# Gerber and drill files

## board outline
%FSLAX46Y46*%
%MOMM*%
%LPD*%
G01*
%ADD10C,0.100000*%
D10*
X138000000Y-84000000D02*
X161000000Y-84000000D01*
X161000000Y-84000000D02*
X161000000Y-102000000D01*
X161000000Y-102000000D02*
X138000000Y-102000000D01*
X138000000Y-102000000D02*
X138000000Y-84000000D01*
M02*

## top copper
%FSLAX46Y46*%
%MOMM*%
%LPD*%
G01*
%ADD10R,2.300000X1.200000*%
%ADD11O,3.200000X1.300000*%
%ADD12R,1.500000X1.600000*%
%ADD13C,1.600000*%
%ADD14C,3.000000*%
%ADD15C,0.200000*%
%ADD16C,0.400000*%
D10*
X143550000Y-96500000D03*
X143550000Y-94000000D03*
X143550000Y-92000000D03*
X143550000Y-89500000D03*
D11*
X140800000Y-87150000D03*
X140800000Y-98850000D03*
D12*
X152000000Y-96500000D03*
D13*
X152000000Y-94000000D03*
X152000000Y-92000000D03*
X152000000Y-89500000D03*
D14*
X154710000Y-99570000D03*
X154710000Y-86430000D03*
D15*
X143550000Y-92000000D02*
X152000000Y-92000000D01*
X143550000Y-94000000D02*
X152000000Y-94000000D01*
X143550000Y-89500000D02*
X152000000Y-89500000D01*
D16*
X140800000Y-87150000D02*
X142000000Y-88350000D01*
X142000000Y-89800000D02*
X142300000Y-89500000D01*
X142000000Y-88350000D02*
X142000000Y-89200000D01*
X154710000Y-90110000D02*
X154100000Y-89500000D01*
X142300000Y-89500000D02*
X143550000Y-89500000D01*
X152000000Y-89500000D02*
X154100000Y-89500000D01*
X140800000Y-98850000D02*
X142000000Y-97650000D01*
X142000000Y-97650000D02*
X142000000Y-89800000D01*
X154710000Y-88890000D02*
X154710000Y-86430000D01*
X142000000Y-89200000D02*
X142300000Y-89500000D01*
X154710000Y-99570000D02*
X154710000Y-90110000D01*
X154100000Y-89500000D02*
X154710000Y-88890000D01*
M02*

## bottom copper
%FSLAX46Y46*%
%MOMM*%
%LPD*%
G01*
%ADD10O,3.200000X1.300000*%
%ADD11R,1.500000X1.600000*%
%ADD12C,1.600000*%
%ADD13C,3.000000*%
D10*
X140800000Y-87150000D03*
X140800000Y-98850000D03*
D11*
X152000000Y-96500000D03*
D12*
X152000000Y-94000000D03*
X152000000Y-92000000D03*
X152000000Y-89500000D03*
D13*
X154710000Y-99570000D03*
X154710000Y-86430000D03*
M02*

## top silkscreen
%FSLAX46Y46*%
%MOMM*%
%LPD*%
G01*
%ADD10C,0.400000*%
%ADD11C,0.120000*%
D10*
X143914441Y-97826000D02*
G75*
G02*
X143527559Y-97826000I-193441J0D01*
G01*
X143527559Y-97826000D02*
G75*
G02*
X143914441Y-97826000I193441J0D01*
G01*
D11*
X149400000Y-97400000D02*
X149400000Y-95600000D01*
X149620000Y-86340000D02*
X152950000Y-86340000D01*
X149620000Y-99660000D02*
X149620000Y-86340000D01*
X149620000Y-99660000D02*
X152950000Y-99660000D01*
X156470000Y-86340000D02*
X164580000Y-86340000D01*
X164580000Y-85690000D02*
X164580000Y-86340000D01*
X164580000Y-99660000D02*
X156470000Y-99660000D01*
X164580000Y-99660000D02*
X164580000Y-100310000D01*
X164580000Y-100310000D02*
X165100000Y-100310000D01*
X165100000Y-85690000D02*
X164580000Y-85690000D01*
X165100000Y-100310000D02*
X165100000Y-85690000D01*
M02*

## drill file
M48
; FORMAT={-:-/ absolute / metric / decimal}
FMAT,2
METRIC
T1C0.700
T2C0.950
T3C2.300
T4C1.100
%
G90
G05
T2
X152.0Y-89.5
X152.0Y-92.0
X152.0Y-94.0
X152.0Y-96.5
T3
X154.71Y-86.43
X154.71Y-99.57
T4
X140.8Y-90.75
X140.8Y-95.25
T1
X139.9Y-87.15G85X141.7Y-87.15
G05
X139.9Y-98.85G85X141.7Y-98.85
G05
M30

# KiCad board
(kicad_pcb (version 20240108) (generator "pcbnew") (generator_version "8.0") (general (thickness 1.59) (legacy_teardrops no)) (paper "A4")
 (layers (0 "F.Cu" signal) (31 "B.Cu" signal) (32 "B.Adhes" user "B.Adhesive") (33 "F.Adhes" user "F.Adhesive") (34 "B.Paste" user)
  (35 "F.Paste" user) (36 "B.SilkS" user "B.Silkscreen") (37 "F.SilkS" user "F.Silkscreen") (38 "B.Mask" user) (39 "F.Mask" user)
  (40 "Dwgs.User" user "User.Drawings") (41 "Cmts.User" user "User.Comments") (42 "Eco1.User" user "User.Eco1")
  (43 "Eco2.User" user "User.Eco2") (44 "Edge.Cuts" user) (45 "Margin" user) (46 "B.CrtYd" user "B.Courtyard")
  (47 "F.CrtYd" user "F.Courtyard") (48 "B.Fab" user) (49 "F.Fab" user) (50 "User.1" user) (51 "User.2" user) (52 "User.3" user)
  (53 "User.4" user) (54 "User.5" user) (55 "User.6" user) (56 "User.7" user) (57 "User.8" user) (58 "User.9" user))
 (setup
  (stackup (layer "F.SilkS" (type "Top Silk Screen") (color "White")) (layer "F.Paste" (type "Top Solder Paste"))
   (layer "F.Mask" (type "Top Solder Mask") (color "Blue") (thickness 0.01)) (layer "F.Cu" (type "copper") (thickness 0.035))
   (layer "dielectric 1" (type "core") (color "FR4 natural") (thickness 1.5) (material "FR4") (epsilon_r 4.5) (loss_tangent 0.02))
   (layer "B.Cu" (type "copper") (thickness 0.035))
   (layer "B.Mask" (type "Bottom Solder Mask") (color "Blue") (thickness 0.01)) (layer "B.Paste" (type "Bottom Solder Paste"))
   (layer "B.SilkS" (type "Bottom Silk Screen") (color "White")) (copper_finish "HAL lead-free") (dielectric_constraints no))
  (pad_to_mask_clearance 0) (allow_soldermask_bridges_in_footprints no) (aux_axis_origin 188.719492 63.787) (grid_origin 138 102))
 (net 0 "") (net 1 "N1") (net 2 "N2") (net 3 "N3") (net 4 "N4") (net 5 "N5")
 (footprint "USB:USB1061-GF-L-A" (layer "F.Cu") (at 140.8 93 -90)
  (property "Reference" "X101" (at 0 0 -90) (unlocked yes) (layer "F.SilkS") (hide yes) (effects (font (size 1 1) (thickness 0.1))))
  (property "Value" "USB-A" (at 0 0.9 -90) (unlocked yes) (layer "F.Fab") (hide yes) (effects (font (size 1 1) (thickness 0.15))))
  (fp_circle (center 4.826 -2.921) (end 5.019441 -2.921) (stroke (width 0.4) (type solid)) (fill none) (layer "F.SilkS"))
  (pad "" np_thru_hole circle (at -2.25 0 270) (size 1.1 1.1) (drill 1.1) (layers "*.Cu" "*.Mask"))
  (pad "" np_thru_hole circle (at 2.25 0 270) (size 1.1 1.1) (drill 1.1) (layers "*.Cu" "*.Mask"))
  (pad "1" smd rect (at 3.5 -2.75 270) (size 1.2 2.3) (layers "F.Cu" "F.Paste" "F.Mask") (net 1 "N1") (solder_mask_margin 0.102))
  (pad "2" smd rect (at 1 -2.75 270) (size 1.2 2.3) (layers "F.Cu" "F.Paste" "F.Mask") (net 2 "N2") (solder_mask_margin 0.102))
  (pad "3" smd rect (at -1 -2.75 270) (size 1.2 2.3) (layers "F.Cu" "F.Paste" "F.Mask") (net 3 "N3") (solder_mask_margin 0.102))
  (pad "4" smd rect (at -3.5 -2.75 270) (size 1.2 2.3) (layers "F.Cu" "F.Paste" "F.Mask") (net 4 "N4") (solder_mask_margin 0.102))
  (pad "5" thru_hole oval (at -5.85 0) (size 3.2 1.3) (drill oval 2.5 0.7) (layers "*.Cu" "*.Mask") (remove_unused_layers no) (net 4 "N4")
   (thermal_bridge_angle 45))
  (pad "5" thru_hole oval (at 5.85 0) (size 3.2 1.3) (drill oval 2.5 0.7) (layers "*.Cu" "*.Mask") (remove_unused_layers no) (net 4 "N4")
   (thermal_bridge_angle 45)))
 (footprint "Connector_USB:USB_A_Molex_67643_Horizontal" (layer "F.Cu") (at 152 96.5 90)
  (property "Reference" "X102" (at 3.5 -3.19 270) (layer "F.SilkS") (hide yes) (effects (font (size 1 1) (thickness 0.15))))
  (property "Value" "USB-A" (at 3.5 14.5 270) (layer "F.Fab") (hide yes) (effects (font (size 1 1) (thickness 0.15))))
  (fp_line (start -0.9 -2.6) (end 0.9 -2.6) (stroke (width 0.12) (type solid)) (layer "F.SilkS"))
  (fp_line (start 10.16 -2.38) (end 10.16 0.95) (stroke (width 0.12) (type solid)) (layer "F.SilkS"))
  (fp_line (start -3.16 -2.38) (end 10.16 -2.38) (stroke (width 0.12) (type solid)) (layer "F.SilkS"))
  (fp_line (start -3.16 -2.38) (end -3.16 0.95) (stroke (width 0.12) (type solid)) (layer "F.SilkS"))
  (fp_line (start 10.16 4.47) (end 10.16 12.58) (stroke (width 0.12) (type solid)) (layer "F.SilkS"))
  (fp_line (start 10.81 12.58) (end 10.16 12.58) (stroke (width 0.12) (type solid)) (layer "F.SilkS"))
  (fp_line (start -3.16 12.58) (end -3.16 4.47) (stroke (width 0.12) (type solid)) (layer "F.SilkS"))
  (fp_line (start -3.16 12.58) (end -3.81 12.58) (stroke (width 0.12) (type solid)) (layer "F.SilkS"))
  (fp_line (start -3.81 12.58) (end -3.81 13.1) (stroke (width 0.12) (type solid)) (layer "F.SilkS"))
  (fp_line (start 10.81 13.1) (end 10.81 12.58) (stroke (width 0.12) (type solid)) (layer "F.SilkS"))
  (fp_line (start -3.81 13.1) (end 10.81 13.1) (stroke (width 0.12) (type solid)) (layer "F.SilkS"))
  (pad "1" thru_hole rect (at 0 0 90) (size 1.6 1.5) (drill 0.95) (layers "*.Cu" "*.Mask") (remove_unused_layers no) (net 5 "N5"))
  (pad "2" thru_hole circle (at 2.5 0 90) (size 1.6 1.6) (drill 0.95) (layers "*.Cu" "*.Mask") (remove_unused_layers no) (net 2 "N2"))
  (pad "3" thru_hole circle (at 4.5 0 90) (size 1.6 1.6) (drill 0.95) (layers "*.Cu" "*.Mask") (remove_unused_layers no) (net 3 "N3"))
  (pad "4" thru_hole circle (at 7 0 90) (size 1.6 1.6) (drill 0.95) (layers "*.Cu" "*.Mask") (remove_unused_layers no) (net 4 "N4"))
  (pad "5" thru_hole circle (at -3.07 2.71 90) (size 3 3) (drill 2.3) (layers "*.Cu" "*.Mask") (remove_unused_layers no) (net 4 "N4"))
  (pad "5" thru_hole circle (at 10.07 2.71 90) (size 3 3) (drill 2.3) (layers "*.Cu" "*.Mask") (remove_unused_layers no) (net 4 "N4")))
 (gr_line (start 138 84) (end 161 84) (stroke (width 0.1) (type default)) (layer "Edge.Cuts"))
 (gr_line (start 161 84) (end 161 102) (stroke (width 0.1) (type default)) (layer "Edge.Cuts"))
 (gr_line (start 161 102) (end 138 102) (stroke (width 0.1) (type default)) (layer "Edge.Cuts"))
 (gr_line (start 138 102) (end 138 84) (stroke (width 0.1) (type default)) (layer "Edge.Cuts"))
 (segment (start 143.55 92) (end 152 92) (width 0.2) (layer "F.Cu") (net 3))
 (segment (start 143.55 94) (end 152 94) (width 0.2) (layer "F.Cu") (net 2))
 (segment (start 143.55 89.5) (end 152 89.5) (width 0.2) (layer "F.Cu") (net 4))
 (segment (start 140.8 87.15) (end 142 88.35) (width 0.4) (layer "F.Cu") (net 4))
 (segment (start 142 89.8) (end 142.3 89.5) (width 0.4) (layer "F.Cu") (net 4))
 (segment (start 142 88.35) (end 142 89.2) (width 0.4) (layer "F.Cu") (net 4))
 (segment (start 154.71 90.11) (end 154.1 89.5) (width 0.4) (layer "F.Cu") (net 4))
 (segment (start 142.3 89.5) (end 143.55 89.5) (width 0.4) (layer "F.Cu") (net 4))
 (segment (start 152 89.5) (end 154.1 89.5) (width 0.4) (layer "F.Cu") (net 4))
 (segment (start 140.8 98.85) (end 142 97.65) (width 0.4) (layer "F.Cu") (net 4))
 (segment (start 142 97.65) (end 142 89.8) (width 0.4) (layer "F.Cu") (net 4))
 (segment (start 154.71 88.89) (end 154.71 86.43) (width 0.4) (layer "F.Cu") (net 4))
 (segment (start 142 89.2) (end 142.3 89.5) (width 0.4) (layer "F.Cu") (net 4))
 (segment (start 154.71 99.57) (end 154.71 90.11) (width 0.4) (layer "F.Cu") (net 4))
 (segment (start 154.1 89.5) (end 154.71 88.89) (width 0.4) (layer "F.Cu") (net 4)))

